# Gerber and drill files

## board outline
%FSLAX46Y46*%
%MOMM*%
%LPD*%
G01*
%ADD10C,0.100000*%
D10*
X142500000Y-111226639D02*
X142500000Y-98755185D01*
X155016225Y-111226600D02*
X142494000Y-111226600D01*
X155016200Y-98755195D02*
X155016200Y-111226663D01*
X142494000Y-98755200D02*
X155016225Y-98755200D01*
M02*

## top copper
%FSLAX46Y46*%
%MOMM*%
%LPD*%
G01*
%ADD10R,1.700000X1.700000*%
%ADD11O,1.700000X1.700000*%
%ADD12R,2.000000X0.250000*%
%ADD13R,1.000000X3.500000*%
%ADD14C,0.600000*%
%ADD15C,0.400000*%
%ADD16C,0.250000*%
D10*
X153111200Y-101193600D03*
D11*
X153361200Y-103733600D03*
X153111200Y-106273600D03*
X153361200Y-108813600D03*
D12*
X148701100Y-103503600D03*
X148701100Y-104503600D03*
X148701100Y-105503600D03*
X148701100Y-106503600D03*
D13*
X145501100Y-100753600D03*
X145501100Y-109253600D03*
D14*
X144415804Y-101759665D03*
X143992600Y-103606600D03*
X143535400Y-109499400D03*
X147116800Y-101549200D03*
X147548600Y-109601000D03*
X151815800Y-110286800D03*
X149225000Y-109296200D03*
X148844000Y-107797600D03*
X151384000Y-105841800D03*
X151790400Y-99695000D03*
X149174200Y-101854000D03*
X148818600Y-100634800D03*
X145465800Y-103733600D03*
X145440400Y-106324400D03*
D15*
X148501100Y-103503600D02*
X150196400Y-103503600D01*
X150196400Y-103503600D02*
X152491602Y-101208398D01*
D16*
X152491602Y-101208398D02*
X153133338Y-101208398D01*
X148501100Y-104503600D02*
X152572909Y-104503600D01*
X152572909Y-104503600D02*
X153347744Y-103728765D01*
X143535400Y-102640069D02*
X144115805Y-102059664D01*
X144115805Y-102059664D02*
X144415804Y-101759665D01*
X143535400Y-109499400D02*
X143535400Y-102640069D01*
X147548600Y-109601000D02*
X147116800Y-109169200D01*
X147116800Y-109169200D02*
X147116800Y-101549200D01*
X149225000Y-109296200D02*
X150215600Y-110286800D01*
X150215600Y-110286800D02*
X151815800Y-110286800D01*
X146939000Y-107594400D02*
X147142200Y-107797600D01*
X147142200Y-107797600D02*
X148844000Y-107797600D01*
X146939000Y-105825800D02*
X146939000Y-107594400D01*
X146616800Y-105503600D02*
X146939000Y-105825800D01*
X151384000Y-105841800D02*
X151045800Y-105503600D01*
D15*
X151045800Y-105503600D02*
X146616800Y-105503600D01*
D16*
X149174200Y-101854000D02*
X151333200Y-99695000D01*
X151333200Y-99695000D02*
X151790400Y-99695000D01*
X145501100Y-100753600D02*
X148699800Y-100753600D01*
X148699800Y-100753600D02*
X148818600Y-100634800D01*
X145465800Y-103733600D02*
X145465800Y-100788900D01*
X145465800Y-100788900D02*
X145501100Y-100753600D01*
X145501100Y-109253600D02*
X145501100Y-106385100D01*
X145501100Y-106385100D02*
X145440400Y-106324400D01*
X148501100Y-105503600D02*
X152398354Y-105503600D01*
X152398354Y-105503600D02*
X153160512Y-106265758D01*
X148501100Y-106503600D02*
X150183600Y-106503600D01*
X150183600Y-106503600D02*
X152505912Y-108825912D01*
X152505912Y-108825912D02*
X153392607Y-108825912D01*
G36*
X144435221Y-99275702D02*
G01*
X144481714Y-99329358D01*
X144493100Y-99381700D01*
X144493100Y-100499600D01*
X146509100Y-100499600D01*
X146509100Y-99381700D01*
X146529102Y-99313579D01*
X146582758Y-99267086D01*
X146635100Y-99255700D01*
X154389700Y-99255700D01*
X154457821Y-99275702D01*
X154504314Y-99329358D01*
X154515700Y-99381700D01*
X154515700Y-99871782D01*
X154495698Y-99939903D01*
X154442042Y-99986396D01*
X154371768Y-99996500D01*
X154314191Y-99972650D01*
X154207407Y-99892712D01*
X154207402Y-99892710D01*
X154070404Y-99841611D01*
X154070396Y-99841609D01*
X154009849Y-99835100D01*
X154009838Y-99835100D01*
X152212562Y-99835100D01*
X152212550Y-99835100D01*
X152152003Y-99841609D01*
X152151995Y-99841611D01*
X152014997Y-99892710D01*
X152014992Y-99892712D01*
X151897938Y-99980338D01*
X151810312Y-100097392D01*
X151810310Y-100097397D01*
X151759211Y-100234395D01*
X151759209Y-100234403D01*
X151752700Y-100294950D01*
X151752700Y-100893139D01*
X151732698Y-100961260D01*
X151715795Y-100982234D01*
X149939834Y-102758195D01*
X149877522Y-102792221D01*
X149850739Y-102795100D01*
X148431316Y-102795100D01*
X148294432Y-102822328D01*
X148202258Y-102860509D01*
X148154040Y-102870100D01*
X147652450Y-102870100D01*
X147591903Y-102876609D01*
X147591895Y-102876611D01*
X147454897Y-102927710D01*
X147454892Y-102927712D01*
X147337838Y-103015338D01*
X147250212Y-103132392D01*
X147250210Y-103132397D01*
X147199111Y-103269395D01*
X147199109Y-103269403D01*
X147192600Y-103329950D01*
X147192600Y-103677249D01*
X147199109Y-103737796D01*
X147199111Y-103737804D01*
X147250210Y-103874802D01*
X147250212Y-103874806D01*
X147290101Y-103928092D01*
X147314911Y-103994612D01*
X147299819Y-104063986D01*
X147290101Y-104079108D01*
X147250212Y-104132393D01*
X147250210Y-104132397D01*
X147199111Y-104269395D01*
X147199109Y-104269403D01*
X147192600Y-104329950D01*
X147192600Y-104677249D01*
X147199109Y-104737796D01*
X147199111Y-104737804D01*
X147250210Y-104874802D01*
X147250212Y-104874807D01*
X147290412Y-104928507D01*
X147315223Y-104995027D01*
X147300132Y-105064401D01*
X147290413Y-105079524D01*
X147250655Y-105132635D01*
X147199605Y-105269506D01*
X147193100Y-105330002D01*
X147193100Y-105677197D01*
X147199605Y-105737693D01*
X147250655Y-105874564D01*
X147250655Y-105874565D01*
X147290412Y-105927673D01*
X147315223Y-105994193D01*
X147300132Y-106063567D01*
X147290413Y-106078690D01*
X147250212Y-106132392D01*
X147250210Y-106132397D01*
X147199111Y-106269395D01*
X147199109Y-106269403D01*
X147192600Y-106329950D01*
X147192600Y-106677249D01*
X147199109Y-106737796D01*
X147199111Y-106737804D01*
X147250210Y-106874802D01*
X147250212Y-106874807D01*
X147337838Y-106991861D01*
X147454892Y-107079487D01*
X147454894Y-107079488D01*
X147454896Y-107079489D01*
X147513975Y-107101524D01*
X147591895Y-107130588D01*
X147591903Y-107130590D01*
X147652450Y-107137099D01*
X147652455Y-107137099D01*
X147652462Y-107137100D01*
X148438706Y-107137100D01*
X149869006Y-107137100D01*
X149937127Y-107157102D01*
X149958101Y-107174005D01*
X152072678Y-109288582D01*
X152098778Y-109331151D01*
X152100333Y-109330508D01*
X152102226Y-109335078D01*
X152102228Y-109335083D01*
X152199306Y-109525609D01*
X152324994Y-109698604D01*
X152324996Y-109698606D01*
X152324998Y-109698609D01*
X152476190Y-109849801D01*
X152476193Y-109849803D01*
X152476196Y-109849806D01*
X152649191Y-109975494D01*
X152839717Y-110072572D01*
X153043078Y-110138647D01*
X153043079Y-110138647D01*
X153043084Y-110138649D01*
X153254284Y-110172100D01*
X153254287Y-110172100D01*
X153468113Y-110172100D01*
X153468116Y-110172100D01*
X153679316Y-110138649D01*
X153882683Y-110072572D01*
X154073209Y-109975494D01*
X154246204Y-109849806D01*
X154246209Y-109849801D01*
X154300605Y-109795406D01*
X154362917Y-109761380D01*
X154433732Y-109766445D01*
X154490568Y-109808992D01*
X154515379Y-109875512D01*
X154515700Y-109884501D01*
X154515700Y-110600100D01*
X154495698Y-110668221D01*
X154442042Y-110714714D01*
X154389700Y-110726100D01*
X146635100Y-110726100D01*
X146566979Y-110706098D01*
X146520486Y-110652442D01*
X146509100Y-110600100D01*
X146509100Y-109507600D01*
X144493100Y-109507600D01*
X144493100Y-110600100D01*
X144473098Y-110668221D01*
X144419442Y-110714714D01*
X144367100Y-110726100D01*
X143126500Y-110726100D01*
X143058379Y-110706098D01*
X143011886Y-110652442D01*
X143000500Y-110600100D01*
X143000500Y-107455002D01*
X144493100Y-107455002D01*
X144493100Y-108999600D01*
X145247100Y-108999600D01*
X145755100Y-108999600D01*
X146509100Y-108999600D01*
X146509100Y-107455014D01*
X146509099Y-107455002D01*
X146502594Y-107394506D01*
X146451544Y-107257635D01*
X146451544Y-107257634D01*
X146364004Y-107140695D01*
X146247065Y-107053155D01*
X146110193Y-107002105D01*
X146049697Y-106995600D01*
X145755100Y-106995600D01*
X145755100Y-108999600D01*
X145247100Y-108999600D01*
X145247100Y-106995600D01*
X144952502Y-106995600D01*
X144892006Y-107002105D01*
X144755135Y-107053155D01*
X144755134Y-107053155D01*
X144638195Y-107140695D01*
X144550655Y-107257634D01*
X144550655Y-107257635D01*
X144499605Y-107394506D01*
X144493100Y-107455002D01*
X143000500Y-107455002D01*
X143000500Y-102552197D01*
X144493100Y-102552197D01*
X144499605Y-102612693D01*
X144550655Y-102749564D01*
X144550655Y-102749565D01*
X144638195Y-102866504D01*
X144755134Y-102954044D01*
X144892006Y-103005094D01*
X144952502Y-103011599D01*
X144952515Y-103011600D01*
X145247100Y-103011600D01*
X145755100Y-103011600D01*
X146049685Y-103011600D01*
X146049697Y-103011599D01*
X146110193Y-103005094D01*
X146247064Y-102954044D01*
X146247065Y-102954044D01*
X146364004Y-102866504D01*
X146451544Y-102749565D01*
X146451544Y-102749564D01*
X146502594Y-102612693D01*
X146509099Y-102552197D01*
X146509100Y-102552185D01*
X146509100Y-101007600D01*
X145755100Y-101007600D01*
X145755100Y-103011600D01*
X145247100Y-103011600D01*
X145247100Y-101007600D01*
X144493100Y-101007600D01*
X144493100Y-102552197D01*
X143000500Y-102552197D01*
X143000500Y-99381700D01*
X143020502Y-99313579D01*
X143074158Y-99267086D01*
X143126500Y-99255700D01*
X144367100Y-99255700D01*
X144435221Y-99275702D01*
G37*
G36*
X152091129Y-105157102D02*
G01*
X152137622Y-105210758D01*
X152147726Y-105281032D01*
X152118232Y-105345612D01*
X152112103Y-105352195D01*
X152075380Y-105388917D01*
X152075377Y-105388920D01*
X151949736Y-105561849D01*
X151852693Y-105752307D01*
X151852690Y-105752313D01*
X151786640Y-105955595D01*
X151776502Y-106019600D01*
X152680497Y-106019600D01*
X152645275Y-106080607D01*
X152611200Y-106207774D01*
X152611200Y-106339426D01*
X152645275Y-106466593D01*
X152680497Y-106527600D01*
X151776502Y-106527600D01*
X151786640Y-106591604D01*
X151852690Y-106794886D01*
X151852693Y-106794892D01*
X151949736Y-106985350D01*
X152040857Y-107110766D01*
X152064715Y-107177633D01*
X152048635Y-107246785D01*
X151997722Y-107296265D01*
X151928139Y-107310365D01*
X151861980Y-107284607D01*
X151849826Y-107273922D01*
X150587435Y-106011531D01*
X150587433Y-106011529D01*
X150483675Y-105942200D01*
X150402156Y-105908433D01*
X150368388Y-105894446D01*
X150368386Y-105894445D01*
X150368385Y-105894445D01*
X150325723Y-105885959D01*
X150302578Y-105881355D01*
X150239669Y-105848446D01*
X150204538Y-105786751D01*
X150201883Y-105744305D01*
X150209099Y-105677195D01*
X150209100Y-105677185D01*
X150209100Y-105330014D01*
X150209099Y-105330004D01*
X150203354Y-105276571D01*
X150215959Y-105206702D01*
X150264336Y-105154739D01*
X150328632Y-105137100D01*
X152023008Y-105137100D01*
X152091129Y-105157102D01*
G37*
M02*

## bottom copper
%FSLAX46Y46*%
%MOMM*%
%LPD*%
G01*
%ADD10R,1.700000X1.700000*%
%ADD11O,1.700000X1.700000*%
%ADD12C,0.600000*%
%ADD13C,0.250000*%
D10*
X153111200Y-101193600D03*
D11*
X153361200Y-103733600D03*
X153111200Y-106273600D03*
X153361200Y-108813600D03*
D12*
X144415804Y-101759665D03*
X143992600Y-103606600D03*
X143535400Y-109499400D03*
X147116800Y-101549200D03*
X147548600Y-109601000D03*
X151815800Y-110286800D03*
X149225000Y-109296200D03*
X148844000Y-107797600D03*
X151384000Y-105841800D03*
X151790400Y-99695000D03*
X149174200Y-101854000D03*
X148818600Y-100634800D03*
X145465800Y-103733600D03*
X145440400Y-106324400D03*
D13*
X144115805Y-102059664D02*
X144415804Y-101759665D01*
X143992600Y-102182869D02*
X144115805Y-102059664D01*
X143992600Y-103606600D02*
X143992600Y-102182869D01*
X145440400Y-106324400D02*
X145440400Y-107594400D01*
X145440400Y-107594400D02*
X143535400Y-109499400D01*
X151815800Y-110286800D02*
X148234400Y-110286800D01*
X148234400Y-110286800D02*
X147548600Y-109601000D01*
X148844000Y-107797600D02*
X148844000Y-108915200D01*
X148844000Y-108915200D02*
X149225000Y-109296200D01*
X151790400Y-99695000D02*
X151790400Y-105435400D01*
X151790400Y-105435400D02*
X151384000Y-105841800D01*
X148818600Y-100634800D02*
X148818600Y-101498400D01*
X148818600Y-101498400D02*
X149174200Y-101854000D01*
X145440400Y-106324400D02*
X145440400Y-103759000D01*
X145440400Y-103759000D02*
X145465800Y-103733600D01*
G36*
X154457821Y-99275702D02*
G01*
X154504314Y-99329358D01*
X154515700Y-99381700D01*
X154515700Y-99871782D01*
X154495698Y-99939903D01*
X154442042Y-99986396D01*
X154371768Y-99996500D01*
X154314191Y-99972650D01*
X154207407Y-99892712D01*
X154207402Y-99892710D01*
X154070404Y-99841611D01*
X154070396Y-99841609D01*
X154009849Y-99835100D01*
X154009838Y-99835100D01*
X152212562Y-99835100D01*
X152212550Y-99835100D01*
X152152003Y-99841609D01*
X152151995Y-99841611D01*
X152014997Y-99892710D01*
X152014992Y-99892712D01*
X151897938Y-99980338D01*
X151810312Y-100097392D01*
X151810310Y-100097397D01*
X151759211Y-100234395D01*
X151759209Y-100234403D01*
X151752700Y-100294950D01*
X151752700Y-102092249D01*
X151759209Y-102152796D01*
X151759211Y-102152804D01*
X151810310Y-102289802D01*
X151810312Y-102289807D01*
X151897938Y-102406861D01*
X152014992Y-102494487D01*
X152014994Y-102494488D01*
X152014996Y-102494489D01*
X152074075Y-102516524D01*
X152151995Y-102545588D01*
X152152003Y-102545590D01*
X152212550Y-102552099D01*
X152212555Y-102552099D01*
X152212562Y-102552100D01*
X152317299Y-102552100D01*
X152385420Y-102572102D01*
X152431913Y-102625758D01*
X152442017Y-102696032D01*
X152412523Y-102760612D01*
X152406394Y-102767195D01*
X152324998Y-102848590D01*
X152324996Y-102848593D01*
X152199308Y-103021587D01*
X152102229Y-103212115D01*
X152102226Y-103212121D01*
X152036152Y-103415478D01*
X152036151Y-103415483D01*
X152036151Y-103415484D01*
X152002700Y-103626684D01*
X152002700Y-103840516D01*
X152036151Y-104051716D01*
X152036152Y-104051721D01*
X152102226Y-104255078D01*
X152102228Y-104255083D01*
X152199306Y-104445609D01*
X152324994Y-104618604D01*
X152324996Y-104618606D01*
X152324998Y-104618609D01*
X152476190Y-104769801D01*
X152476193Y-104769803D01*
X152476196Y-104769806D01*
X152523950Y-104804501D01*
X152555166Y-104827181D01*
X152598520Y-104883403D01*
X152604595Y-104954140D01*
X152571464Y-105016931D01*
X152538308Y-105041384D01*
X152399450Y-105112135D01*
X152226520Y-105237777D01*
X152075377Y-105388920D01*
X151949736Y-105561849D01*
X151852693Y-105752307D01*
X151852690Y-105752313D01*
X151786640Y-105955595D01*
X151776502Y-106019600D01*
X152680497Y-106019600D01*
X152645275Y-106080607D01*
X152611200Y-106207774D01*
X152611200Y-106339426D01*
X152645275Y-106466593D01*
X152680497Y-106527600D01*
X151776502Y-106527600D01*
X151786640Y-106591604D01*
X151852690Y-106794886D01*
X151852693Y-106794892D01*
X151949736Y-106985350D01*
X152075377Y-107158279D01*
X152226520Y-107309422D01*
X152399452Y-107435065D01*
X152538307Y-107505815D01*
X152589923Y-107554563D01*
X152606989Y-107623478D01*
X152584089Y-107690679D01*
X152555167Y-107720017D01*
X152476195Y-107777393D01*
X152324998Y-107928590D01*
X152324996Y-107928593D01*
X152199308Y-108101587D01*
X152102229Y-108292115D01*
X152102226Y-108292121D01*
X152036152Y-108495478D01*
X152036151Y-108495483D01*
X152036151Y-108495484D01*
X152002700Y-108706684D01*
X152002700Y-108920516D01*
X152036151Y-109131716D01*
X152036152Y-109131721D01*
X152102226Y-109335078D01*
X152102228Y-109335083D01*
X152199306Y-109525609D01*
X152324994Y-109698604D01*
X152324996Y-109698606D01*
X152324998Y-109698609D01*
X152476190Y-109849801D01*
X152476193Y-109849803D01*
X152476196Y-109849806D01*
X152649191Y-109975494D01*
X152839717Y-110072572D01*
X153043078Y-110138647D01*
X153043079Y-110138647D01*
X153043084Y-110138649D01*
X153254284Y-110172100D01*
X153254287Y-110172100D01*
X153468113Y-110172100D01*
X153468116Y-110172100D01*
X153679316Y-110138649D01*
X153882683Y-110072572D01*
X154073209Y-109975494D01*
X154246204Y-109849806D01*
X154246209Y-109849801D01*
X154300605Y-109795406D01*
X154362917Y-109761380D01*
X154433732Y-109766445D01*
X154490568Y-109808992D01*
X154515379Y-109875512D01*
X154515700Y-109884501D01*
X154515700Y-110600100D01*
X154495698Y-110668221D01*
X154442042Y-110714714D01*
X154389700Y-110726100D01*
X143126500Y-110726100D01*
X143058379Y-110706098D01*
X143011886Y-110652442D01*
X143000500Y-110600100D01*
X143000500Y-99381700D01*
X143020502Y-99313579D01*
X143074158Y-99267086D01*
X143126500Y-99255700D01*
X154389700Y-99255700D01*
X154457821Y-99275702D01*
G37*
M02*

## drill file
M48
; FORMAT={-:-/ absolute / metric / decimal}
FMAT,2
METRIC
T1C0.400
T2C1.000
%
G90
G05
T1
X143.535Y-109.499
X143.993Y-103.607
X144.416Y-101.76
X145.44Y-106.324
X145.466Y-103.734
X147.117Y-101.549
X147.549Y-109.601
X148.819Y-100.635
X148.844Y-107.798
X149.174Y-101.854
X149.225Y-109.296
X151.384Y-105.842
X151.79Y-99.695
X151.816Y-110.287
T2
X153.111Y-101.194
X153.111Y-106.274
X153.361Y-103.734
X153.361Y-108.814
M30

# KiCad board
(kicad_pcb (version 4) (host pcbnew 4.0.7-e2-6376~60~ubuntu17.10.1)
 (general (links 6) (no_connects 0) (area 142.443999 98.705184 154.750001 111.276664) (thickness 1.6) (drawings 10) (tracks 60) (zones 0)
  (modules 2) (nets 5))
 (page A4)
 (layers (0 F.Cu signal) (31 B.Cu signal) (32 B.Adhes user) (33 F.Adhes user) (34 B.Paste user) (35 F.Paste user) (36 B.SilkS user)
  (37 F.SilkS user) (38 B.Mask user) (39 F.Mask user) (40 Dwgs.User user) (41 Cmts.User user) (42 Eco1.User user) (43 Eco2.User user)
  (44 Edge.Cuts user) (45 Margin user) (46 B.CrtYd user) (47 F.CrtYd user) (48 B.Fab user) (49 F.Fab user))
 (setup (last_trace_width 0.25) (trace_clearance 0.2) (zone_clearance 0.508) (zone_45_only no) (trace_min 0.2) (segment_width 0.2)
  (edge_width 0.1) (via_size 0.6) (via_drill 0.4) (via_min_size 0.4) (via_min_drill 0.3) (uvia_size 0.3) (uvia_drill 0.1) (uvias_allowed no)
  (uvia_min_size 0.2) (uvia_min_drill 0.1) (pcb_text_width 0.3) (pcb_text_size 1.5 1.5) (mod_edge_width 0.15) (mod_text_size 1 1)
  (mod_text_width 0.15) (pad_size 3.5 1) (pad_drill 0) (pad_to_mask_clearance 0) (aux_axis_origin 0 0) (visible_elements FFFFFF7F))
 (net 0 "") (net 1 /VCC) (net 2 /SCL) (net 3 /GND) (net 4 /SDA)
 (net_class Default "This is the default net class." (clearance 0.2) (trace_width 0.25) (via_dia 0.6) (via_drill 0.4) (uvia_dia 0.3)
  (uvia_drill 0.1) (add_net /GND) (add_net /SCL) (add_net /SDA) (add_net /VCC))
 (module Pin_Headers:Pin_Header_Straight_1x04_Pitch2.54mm (layer F.Cu) (at 153.1112 101.1936)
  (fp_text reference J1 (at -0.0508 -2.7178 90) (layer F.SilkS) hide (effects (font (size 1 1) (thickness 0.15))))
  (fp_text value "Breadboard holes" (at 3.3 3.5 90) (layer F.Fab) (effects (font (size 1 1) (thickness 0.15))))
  (pad 1 thru_hole rect (at 0 0) (size 1.7 1.7) (drill 1) (layers *.Cu *.Mask) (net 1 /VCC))
  (pad 2 thru_hole oval (at 0.25 2.54) (size 1.7 1.7) (drill 1) (layers *.Cu *.Mask) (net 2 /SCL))
  (pad 3 thru_hole oval (at 0 5.08) (size 1.7 1.7) (drill 1) (layers *.Cu *.Mask) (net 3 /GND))
  (pad 4 thru_hole oval (at 0.25 7.62) (size 1.7 1.7) (drill 1) (layers *.Cu *.Mask) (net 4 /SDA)))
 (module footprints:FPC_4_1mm (layer F.Cu) (at 148.5011 105.0036 270)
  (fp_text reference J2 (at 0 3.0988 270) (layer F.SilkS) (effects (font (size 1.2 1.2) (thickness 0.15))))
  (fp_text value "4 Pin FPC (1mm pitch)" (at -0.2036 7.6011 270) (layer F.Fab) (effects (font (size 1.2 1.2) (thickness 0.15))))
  (pad 1 smd rect (at -1.5 -0.2 270) (size 0.25 2) (layers F.Cu F.Paste F.Mask) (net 1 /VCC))
  (pad 2 smd rect (at -0.5 -0.2 270) (size 0.25 2) (layers F.Cu F.Paste F.Mask) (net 2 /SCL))
  (pad 3 smd rect (at 0.5 -0.2 270) (size 0.25 2) (layers F.Cu F.Paste F.Mask) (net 3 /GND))
  (pad 4 smd rect (at 1.5 -0.2 270) (size 0.25 2) (layers F.Cu F.Paste F.Mask) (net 4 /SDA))
  (pad 0 smd rect (at -4.25 3 270) (size 3.5 1) (layers F.Cu F.Paste F.Mask) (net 3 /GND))
  (pad 0 smd rect (at 4.25 3 270) (size 3.5 1) (layers F.Cu F.Paste F.Mask) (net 3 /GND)))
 (gr_line (start 142.5 111.226639) (end 142.5 98.755185) (angle 90) (layer Edge.Cuts) (width 0.1))
 (gr_line (start 155.016225 111.2266) (end 142.494 111.2266) (angle 90) (layer Edge.Cuts) (width 0.1))
 (gr_line (start 155.0162 98.755195) (end 155.0162 111.226663) (angle 90) (layer Edge.Cuts) (width 0.1))
 (gr_line (start 142.494 98.7552) (end 155.016225 98.7552) (angle 90) (layer Edge.Cuts) (width 0.1))
 (segment (start 148.5011 103.5036) (end 150.1964 103.5036) (width 0.4) (layer F.Cu) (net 1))
 (segment (start 150.1964 103.5036) (end 152.491602 101.208398) (width 0.4) (layer F.Cu) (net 1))
 (segment (start 152.491602 101.208398) (end 153.133338 101.208398) (width 0.25) (layer F.Cu) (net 1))
 (segment (start 148.5011 104.5036) (end 152.572909 104.5036) (width 0.25) (layer F.Cu) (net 2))
 (segment (start 152.572909 104.5036) (end 153.347744 103.728765) (width 0.25) (layer F.Cu) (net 2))
 (segment (start 144.115805 102.059664) (end 144.415804 101.759665) (width 0.25) (layer B.Cu) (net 3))
 (segment (start 143.9926 102.182869) (end 144.115805 102.059664) (width 0.25) (layer B.Cu) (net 3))
 (segment (start 143.5354 102.640069) (end 144.115805 102.059664) (width 0.25) (layer F.Cu) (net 3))
 (segment (start 143.9926 103.6066) (end 143.9926 102.182869) (width 0.25) (layer B.Cu) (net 3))
 (segment (start 144.115805 102.059664) (end 144.415804 101.759665) (width 0.25) (layer F.Cu) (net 3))
 (segment (start 143.5354 109.4994) (end 143.5354 102.640069) (width 0.25) (layer F.Cu) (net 3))
 (via (at 144.415804 101.759665) (size 0.6) (drill 0.4) (layers F.Cu B.Cu) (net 3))
 (via (at 143.9926 103.6066) (size 0.6) (drill 0.4) (layers F.Cu B.Cu) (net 3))
 (segment (start 145.4404 106.3244) (end 145.4404 107.5944) (width 0.25) (layer B.Cu) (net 3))
 (segment (start 145.4404 107.5944) (end 143.5354 109.4994) (width 0.25) (layer B.Cu) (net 3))
 (via (at 143.5354 109.4994) (size 0.6) (drill 0.4) (layers F.Cu B.Cu) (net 3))
 (segment (start 147.5486 109.601) (end 147.1168 109.1692) (width 0.25) (layer F.Cu) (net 3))
 (segment (start 147.1168 109.1692) (end 147.1168 101.5492) (width 0.25) (layer F.Cu) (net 3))
 (via (at 147.1168 101.5492) (size 0.6) (drill 0.4) (layers F.Cu B.Cu) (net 3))
 (segment (start 151.8158 110.2868) (end 148.2344 110.2868) (width 0.25) (layer B.Cu) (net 3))
 (segment (start 148.2344 110.2868) (end 147.5486 109.601) (width 0.25) (layer B.Cu) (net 3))
 (via (at 147.5486 109.601) (size 0.6) (drill 0.4) (layers F.Cu B.Cu) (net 3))
 (segment (start 149.225 109.2962) (end 150.2156 110.2868) (width 0.25) (layer F.Cu) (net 3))
 (segment (start 150.2156 110.2868) (end 151.8158 110.2868) (width 0.25) (layer F.Cu) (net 3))
 (via (at 151.8158 110.2868) (size 0.6) (drill 0.4) (layers F.Cu B.Cu) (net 3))
 (segment (start 148.844 107.7976) (end 148.844 108.9152) (width 0.25) (layer B.Cu) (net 3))
 (segment (start 148.844 108.9152) (end 149.225 109.2962) (width 0.25) (layer B.Cu) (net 3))
 (via (at 149.225 109.2962) (size 0.6) (drill 0.4) (layers F.Cu B.Cu) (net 3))
 (segment (start 146.939 107.5944) (end 147.1422 107.7976) (width 0.25) (layer F.Cu) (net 3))
 (segment (start 147.1422 107.7976) (end 148.844 107.7976) (width 0.25) (layer F.Cu) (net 3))
 (via (at 148.844 107.7976) (size 0.6) (drill 0.4) (layers F.Cu B.Cu) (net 3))
 (segment (start 146.939 105.8258) (end 146.939 107.5944) (width 0.25) (layer F.Cu) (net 3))
 (segment (start 146.6168 105.5036) (end 146.939 105.8258) (width 0.25) (layer F.Cu) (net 3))
 (segment (start 151.384 105.8418) (end 151.0458 105.5036) (width 0.25) (layer F.Cu) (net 3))
 (segment (start 151.0458 105.5036) (end 146.6168 105.5036) (width 0.4) (layer F.Cu) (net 3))
 (segment (start 151.7904 99.695) (end 151.7904 105.4354) (width 0.25) (layer B.Cu) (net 3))
 (segment (start 151.7904 105.4354) (end 151.384 105.8418) (width 0.25) (layer B.Cu) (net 3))
 (via (at 151.384 105.8418) (size 0.6) (drill 0.4) (layers F.Cu B.Cu) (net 3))
 (segment (start 149.1742 101.854) (end 151.3332 99.695) (width 0.25) (layer F.Cu) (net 3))
 (segment (start 151.3332 99.695) (end 151.7904 99.695) (width 0.25) (layer F.Cu) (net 3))
 (via (at 151.7904 99.695) (size 0.6) (drill 0.4) (layers F.Cu B.Cu) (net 3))
 (segment (start 148.8186 100.6348) (end 148.8186 101.4984) (width 0.25) (layer B.Cu) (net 3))
 (segment (start 148.8186 101.4984) (end 149.1742 101.854) (width 0.25) (layer B.Cu) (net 3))
 (via (at 149.1742 101.854) (size 0.6) (drill 0.4) (layers F.Cu B.Cu) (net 3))
 (segment (start 145.5011 100.7536) (end 148.6998 100.7536) (width 0.25) (layer F.Cu) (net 3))
 (segment (start 148.6998 100.7536) (end 148.8186 100.6348) (width 0.25) (layer F.Cu) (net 3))
 (via (at 148.8186 100.6348) (size 0.6) (drill 0.4) (layers F.Cu B.Cu) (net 3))
 (segment (start 145.4658 103.7336) (end 145.4658 100.7889) (width 0.25) (layer F.Cu) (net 3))
 (segment (start 145.4658 100.7889) (end 145.5011 100.7536) (width 0.25) (layer F.Cu) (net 3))
 (segment (start 145.4404 106.3244) (end 145.4404 103.759) (width 0.25) (layer B.Cu) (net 3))
 (segment (start 145.4404 103.759) (end 145.4658 103.7336) (width 0.25) (layer B.Cu) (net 3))
 (via (at 145.4658 103.7336) (size 0.6) (drill 0.4) (layers F.Cu B.Cu) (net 3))
 (segment (start 145.5011 109.2536) (end 145.5011 106.3851) (width 0.25) (layer F.Cu) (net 3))
 (segment (start 145.5011 106.3851) (end 145.4404 106.3244) (width 0.25) (layer F.Cu) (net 3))
 (via (at 145.4404 106.3244) (size 0.6) (drill 0.4) (layers F.Cu B.Cu) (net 3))
 (segment (start 148.5011 105.5036) (end 152.398354 105.5036) (width 0.25) (layer F.Cu) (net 3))
 (segment (start 152.398354 105.5036) (end 153.160512 106.265758) (width 0.25) (layer F.Cu) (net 3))
 (segment (start 148.5011 106.5036) (end 150.1836 106.5036) (width 0.25) (layer F.Cu) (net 4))
 (segment (start 150.1836 106.5036) (end 152.505912 108.825912) (width 0.25) (layer F.Cu) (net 4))
 (segment (start 152.505912 108.825912) (end 153.392607 108.825912) (width 0.25) (layer F.Cu) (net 4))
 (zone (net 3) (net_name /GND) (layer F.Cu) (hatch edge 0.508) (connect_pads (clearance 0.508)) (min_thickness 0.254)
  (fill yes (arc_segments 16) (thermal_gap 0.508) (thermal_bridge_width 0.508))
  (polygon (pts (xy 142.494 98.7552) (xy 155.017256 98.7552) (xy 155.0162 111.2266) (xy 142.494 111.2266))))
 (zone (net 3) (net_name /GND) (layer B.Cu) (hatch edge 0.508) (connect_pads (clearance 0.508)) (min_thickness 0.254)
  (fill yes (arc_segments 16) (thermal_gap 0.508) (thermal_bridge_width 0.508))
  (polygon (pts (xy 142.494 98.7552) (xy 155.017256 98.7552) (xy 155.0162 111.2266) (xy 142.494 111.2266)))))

